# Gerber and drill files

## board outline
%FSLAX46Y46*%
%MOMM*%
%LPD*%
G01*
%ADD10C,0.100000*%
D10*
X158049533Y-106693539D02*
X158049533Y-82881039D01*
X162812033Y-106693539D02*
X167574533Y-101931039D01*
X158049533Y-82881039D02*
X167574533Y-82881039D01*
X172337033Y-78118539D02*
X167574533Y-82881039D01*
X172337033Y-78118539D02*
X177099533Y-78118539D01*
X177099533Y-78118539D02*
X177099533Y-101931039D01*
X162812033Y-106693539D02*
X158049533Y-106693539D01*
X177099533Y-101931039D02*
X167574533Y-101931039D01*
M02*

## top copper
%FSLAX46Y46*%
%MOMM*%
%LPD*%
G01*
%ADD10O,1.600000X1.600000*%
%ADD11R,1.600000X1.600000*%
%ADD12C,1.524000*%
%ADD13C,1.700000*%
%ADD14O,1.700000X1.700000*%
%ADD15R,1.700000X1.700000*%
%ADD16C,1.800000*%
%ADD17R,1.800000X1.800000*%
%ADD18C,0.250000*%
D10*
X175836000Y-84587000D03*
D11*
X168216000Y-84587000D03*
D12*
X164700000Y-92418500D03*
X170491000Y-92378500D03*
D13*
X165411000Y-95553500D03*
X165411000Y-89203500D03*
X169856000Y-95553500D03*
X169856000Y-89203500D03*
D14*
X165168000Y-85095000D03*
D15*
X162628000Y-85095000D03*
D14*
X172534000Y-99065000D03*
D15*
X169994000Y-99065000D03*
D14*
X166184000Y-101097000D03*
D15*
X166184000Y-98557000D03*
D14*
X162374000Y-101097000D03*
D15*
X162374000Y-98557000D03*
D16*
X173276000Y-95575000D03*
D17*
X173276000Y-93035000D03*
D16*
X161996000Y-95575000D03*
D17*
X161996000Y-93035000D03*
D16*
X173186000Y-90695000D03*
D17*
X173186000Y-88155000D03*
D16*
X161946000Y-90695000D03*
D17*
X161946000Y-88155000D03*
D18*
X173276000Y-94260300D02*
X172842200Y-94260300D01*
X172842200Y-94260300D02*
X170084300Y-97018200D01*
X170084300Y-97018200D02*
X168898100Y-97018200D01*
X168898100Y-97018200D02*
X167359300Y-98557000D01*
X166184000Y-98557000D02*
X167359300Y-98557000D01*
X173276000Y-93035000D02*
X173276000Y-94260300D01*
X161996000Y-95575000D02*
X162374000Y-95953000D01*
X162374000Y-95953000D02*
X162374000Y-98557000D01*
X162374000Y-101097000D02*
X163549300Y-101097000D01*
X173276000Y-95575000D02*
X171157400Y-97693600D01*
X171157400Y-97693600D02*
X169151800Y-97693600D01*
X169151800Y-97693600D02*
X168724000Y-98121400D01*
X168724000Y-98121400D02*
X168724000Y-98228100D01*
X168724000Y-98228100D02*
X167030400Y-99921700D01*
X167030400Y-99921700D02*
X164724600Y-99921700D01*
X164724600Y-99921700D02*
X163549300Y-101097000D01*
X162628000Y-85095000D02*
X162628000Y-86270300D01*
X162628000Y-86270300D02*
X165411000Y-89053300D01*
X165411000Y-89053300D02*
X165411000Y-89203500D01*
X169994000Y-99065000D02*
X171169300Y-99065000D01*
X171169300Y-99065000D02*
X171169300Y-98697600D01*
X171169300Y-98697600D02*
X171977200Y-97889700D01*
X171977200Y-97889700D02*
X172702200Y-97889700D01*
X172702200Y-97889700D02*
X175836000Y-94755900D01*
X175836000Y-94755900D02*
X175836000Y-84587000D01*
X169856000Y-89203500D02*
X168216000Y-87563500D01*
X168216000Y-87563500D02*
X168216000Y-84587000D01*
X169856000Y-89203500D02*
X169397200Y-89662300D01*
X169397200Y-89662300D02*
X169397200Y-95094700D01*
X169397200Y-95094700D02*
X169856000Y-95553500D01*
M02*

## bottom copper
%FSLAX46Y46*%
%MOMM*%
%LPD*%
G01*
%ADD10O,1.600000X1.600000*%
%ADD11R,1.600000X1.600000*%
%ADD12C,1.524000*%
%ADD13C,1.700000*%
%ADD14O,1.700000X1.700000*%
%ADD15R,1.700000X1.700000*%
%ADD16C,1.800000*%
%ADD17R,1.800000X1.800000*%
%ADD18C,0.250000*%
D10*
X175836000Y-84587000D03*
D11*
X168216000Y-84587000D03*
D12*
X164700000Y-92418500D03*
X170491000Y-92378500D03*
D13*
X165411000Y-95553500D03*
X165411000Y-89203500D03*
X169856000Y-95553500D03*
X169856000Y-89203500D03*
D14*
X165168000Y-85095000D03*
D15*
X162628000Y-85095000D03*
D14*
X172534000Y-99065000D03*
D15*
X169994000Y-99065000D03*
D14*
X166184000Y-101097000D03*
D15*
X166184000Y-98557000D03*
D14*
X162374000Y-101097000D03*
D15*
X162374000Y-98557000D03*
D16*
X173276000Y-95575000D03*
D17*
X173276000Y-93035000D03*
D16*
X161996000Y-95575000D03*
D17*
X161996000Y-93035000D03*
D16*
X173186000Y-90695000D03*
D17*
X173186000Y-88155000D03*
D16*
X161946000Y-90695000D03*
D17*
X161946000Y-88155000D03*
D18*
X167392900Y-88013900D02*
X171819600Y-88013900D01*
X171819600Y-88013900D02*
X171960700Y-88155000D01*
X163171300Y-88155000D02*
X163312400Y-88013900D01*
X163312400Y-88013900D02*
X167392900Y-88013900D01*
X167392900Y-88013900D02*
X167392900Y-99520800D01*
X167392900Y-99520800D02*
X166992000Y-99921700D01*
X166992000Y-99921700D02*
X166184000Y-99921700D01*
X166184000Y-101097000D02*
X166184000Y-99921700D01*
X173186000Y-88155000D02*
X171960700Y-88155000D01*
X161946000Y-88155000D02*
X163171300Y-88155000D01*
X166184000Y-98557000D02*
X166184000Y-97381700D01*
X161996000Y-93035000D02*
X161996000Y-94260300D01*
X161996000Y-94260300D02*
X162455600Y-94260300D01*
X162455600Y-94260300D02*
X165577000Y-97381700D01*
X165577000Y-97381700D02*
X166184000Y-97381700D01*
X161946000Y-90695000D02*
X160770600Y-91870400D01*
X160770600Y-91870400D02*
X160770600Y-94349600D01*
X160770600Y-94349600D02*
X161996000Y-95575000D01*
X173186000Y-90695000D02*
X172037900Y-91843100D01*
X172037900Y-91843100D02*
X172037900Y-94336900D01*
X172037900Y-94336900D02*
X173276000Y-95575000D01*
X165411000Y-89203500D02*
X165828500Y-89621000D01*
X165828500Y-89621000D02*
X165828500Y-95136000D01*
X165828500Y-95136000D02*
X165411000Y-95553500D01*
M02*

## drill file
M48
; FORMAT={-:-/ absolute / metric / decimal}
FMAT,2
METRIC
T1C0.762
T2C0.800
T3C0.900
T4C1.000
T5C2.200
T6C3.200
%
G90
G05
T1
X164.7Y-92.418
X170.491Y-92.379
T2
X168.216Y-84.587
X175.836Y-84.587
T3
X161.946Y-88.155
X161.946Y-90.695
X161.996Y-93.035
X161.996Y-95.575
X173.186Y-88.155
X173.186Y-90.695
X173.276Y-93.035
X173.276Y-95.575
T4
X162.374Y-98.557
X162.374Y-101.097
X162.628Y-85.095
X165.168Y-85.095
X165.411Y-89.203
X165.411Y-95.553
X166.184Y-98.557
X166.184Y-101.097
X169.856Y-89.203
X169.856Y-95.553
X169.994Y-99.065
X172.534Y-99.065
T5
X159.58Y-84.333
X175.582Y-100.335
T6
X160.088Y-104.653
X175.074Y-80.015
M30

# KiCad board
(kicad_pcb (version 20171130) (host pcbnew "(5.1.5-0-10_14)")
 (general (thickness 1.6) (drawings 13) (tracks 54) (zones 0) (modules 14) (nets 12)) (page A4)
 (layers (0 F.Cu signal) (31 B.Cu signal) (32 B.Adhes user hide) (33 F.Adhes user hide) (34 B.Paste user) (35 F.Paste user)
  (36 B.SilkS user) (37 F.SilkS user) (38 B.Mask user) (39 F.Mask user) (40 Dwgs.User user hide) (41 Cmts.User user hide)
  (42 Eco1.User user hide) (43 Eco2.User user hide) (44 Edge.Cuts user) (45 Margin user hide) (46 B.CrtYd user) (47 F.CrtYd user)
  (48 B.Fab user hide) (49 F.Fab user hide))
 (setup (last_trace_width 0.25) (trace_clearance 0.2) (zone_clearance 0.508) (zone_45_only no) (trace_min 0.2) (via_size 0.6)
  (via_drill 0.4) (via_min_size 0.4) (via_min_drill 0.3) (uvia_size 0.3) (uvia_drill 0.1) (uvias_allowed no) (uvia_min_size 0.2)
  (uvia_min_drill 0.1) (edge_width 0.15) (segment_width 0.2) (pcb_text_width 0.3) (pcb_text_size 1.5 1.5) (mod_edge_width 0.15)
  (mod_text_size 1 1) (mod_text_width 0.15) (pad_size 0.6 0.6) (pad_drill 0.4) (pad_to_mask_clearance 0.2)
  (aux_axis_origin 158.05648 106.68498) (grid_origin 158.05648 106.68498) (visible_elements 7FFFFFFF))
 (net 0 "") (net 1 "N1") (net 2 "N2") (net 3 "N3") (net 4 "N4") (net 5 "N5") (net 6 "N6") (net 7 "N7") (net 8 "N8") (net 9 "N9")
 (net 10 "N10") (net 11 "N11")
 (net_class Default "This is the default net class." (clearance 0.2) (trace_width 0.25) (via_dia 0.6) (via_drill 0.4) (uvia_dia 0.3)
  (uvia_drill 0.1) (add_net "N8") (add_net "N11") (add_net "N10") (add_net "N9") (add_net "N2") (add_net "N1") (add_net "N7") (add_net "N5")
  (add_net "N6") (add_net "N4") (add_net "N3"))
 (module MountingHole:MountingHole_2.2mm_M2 (layer F.Cu) (at 159.58048 84.33298)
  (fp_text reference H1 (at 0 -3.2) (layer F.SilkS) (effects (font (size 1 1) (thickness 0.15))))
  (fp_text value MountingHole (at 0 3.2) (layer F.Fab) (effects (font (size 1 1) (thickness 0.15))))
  (pad 1 np_thru_hole circle (at 0 0) (size 2.2 2.2) (drill 2.2) (layers *.Cu *.Mask)))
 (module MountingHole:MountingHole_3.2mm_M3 (layer F.Cu) (at 160.08848 104.65298)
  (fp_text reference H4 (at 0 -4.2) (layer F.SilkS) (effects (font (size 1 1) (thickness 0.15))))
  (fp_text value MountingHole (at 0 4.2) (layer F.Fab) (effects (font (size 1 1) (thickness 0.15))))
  (pad 1 np_thru_hole circle (at 0 0) (size 3.2 3.2) (drill 3.2) (layers *.Cu *.Mask)))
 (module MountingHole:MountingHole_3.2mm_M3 (layer F.Cu) (at 175.07448 80.01498)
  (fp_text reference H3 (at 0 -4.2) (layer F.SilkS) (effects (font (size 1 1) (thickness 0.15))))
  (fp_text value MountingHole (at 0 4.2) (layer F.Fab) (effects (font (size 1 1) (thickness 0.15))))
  (pad 1 np_thru_hole circle (at 0 0) (size 3.2 3.2) (drill 3.2) (layers *.Cu *.Mask)))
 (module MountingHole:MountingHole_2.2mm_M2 (layer F.Cu) (at 175.58248 100.33498)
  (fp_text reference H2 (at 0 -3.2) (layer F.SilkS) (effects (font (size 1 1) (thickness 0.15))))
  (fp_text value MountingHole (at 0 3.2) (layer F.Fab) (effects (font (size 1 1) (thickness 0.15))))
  (pad 1 np_thru_hole circle (at 0 0) (size 2.2 2.2) (drill 2.2) (layers *.Cu *.Mask)))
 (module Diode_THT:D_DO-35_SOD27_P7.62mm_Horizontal (layer F.Cu) (at 168.216 84.587)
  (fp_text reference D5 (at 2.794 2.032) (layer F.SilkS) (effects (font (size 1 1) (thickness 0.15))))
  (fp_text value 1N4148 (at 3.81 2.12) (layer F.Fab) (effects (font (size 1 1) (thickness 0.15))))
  (pad 2 thru_hole oval (at 7.62 0) (size 1.6 1.6) (drill 0.8) (layers *.Cu *.Mask) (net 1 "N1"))
  (pad 1 thru_hole rect (at 0 0) (size 1.6 1.6) (drill 0.8) (layers *.Cu *.Mask) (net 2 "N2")))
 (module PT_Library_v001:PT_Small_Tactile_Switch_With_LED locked (layer F.Cu) (at 167.57 92.3785 270)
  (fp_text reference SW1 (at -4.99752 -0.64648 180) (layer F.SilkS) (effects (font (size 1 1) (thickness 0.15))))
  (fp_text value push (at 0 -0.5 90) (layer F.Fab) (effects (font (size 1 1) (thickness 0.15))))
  (pad 6 thru_hole circle (at 0.04 2.87 270) (size 1.524 1.524) (drill 0.762) (layers *.Cu *.Mask) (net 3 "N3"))
  (pad 5 thru_hole circle (at 0 -2.921 270) (size 1.524 1.524) (drill 0.762) (layers *.Cu *.Mask) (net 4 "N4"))
  (pad 4 thru_hole circle (at 3.175 2.159 270) (size 1.7 1.7) (drill 1) (layers *.Cu *.Mask) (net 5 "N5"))
  (pad 3 thru_hole circle (at -3.175 2.159 270) (size 1.7 1.7) (drill 1) (layers *.Cu *.Mask) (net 5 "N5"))
  (pad 2 thru_hole circle (at 3.175 -2.286 270) (size 1.7 1.7) (drill 1) (layers *.Cu *.Mask) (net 2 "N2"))
  (pad 1 thru_hole circle (at -3.175 -2.286 270) (size 1.7 1.7) (drill 1) (layers *.Cu *.Mask) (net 2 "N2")))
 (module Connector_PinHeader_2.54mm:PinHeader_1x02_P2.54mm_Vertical (layer B.Cu) (at 162.628 85.095 270)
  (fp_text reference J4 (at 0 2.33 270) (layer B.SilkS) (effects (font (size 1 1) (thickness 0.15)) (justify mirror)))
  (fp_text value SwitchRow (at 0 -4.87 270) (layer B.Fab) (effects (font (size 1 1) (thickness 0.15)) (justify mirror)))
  (pad 2 thru_hole oval (at 0 -2.54 270) (size 1.7 1.7) (drill 1) (layers *.Cu *.Mask) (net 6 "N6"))
  (pad 1 thru_hole rect (at 0 0 270) (size 1.7 1.7) (drill 1) (layers *.Cu *.Mask) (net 5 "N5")))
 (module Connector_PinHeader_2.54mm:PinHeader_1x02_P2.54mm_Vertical (layer B.Cu) (at 169.994 99.065 270)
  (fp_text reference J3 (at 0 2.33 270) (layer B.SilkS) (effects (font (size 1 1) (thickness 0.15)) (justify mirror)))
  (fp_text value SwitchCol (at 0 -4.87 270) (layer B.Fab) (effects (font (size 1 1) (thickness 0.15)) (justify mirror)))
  (pad 2 thru_hole oval (at 0 -2.54 270) (size 1.7 1.7) (drill 1) (layers *.Cu *.Mask) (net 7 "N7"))
  (pad 1 thru_hole rect (at 0 0 270) (size 1.7 1.7) (drill 1) (layers *.Cu *.Mask) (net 1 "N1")))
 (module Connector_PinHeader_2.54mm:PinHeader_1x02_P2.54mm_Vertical (layer B.Cu) (at 166.184 98.557 180)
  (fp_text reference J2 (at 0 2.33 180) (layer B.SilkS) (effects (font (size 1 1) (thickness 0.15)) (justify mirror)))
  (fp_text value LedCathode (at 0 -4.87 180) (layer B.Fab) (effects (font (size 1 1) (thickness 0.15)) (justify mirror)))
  (pad 2 thru_hole oval (at 0 -2.54 180) (size 1.7 1.7) (drill 1) (layers *.Cu *.Mask) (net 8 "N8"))
  (pad 1 thru_hole rect (at 0 0 180) (size 1.7 1.7) (drill 1) (layers *.Cu *.Mask) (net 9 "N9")))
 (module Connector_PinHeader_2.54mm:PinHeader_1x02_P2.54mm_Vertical (layer B.Cu) (at 162.374 98.557 180)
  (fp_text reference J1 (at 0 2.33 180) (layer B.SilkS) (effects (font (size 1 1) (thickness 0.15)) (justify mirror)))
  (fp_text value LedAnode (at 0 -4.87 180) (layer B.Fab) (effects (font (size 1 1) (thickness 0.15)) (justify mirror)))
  (pad 2 thru_hole oval (at 0 -2.54 180) (size 1.7 1.7) (drill 1) (layers *.Cu *.Mask) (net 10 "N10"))
  (pad 1 thru_hole rect (at 0 0 180) (size 1.7 1.7) (drill 1) (layers *.Cu *.Mask) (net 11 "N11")))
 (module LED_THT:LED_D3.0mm (layer F.Cu) (at 173.276 93.035 270)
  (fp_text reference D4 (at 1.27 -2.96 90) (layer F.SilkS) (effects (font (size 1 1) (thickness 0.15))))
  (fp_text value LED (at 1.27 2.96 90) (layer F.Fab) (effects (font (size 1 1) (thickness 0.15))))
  (pad 2 thru_hole circle (at 2.54 0 270) (size 1.8 1.8) (drill 0.9) (layers *.Cu *.Mask) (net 10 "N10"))
  (pad 1 thru_hole rect (at 0 0 270) (size 1.8 1.8) (drill 0.9) (layers *.Cu *.Mask) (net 9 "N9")))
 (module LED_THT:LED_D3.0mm (layer F.Cu) (at 161.996 93.035 270)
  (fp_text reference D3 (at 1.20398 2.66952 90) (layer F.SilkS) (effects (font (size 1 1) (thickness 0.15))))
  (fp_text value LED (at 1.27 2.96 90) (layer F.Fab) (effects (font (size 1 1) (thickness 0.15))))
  (pad 2 thru_hole circle (at 2.54 0 270) (size 1.8 1.8) (drill 0.9) (layers *.Cu *.Mask) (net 11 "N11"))
  (pad 1 thru_hole rect (at 0 0 270) (size 1.8 1.8) (drill 0.9) (layers *.Cu *.Mask) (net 9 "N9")))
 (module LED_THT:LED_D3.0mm (layer F.Cu) (at 173.186 88.155 270)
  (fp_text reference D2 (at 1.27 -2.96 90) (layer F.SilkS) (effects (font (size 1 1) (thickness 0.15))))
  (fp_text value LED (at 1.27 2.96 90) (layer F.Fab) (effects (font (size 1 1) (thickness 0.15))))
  (pad 2 thru_hole circle (at 2.54 0 270) (size 1.8 1.8) (drill 0.9) (layers *.Cu *.Mask) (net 10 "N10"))
  (pad 1 thru_hole rect (at 0 0 270) (size 1.8 1.8) (drill 0.9) (layers *.Cu *.Mask) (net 8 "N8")))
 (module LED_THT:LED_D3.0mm (layer F.Cu) (at 161.946 88.155 270)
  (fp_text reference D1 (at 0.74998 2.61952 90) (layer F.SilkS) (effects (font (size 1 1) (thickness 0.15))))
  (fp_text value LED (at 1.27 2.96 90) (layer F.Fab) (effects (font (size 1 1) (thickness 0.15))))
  (pad 2 thru_hole circle (at 2.54 0 270) (size 1.8 1.8) (drill 0.9) (layers *.Cu *.Mask) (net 11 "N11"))
  (pad 1 thru_hole rect (at 0 0 270) (size 1.8 1.8) (drill 0.9) (layers *.Cu *.Mask) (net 8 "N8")))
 (gr_line (start 158.049533 106.693539) (end 158.049533 82.881039) (layer Edge.Cuts) (width 0.1))
 (gr_line (start 162.812033 106.693539) (end 167.574533 101.931039) (layer Edge.Cuts) (width 0.1))
 (gr_line (start 158.049533 82.881039) (end 167.574533 82.881039) (layer Edge.Cuts) (width 0.1))
 (gr_line (start 172.337033 78.118539) (end 167.574533 82.881039) (layer Edge.Cuts) (width 0.1))
 (gr_line (start 172.337033 78.118539) (end 177.099533 78.118539) (layer Edge.Cuts) (width 0.1))
 (gr_line (start 177.099533 78.118539) (end 177.099533 101.931039) (layer Edge.Cuts) (width 0.1))
 (gr_line (start 162.812033 106.693539) (end 158.049533 106.693539) (layer Edge.Cuts) (width 0.1))
 (gr_line (start 177.099533 101.931039) (end 167.574533 101.931039) (layer Edge.Cuts) (width 0.1))
 (segment (start 167.3929 88.0139) (end 171.8196 88.0139) (width 0.25) (layer B.Cu) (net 8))
 (segment (start 171.8196 88.0139) (end 171.9607 88.155) (width 0.25) (layer B.Cu) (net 8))
 (segment (start 163.1713 88.155) (end 163.3124 88.0139) (width 0.25) (layer B.Cu) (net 8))
 (segment (start 163.3124 88.0139) (end 167.3929 88.0139) (width 0.25) (layer B.Cu) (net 8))
 (segment (start 167.3929 88.0139) (end 167.3929 99.5208) (width 0.25) (layer B.Cu) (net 8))
 (segment (start 167.3929 99.5208) (end 166.992 99.9217) (width 0.25) (layer B.Cu) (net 8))
 (segment (start 166.992 99.9217) (end 166.184 99.9217) (width 0.25) (layer B.Cu) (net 8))
 (segment (start 166.184 101.097) (end 166.184 99.9217) (width 0.25) (layer B.Cu) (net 8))
 (segment (start 173.186 88.155) (end 171.9607 88.155) (width 0.25) (layer B.Cu) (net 8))
 (segment (start 161.946 88.155) (end 163.1713 88.155) (width 0.25) (layer B.Cu) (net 8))
 (segment (start 173.276 94.2603) (end 172.8422 94.2603) (width 0.25) (layer F.Cu) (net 9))
 (segment (start 172.8422 94.2603) (end 170.0843 97.0182) (width 0.25) (layer F.Cu) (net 9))
 (segment (start 170.0843 97.0182) (end 168.8981 97.0182) (width 0.25) (layer F.Cu) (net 9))
 (segment (start 168.8981 97.0182) (end 167.3593 98.557) (width 0.25) (layer F.Cu) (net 9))
 (segment (start 166.184 98.557) (end 167.3593 98.557) (width 0.25) (layer F.Cu) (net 9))
 (segment (start 173.276 93.035) (end 173.276 94.2603) (width 0.25) (layer F.Cu) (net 9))
 (segment (start 166.184 98.557) (end 166.184 97.3817) (width 0.25) (layer B.Cu) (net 9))
 (segment (start 161.996 93.035) (end 161.996 94.2603) (width 0.25) (layer B.Cu) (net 9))
 (segment (start 161.996 94.2603) (end 162.4556 94.2603) (width 0.25) (layer B.Cu) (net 9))
 (segment (start 162.4556 94.2603) (end 165.577 97.3817) (width 0.25) (layer B.Cu) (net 9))
 (segment (start 165.577 97.3817) (end 166.184 97.3817) (width 0.25) (layer B.Cu) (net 9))
 (segment (start 161.996 95.575) (end 162.374 95.953) (width 0.25) (layer F.Cu) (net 11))
 (segment (start 162.374 95.953) (end 162.374 98.557) (width 0.25) (layer F.Cu) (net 11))
 (segment (start 161.946 90.695) (end 160.7706 91.8704) (width 0.25) (layer B.Cu) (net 11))
 (segment (start 160.7706 91.8704) (end 160.7706 94.3496) (width 0.25) (layer B.Cu) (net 11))
 (segment (start 160.7706 94.3496) (end 161.996 95.575) (width 0.25) (layer B.Cu) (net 11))
 (segment (start 162.374 101.097) (end 163.5493 101.097) (width 0.25) (layer F.Cu) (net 10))
 (segment (start 173.276 95.575) (end 171.1574 97.6936) (width 0.25) (layer F.Cu) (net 10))
 (segment (start 171.1574 97.6936) (end 169.1518 97.6936) (width 0.25) (layer F.Cu) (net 10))
 (segment (start 169.1518 97.6936) (end 168.724 98.1214) (width 0.25) (layer F.Cu) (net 10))
 (segment (start 168.724 98.1214) (end 168.724 98.2281) (width 0.25) (layer F.Cu) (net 10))
 (segment (start 168.724 98.2281) (end 167.0304 99.9217) (width 0.25) (layer F.Cu) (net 10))
 (segment (start 167.0304 99.9217) (end 164.7246 99.9217) (width 0.25) (layer F.Cu) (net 10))
 (segment (start 164.7246 99.9217) (end 163.5493 101.097) (width 0.25) (layer F.Cu) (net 10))
 (segment (start 173.186 90.695) (end 172.0379 91.8431) (width 0.25) (layer B.Cu) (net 10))
 (segment (start 172.0379 91.8431) (end 172.0379 94.3369) (width 0.25) (layer B.Cu) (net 10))
 (segment (start 172.0379 94.3369) (end 173.276 95.575) (width 0.25) (layer B.Cu) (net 10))
 (segment (start 162.628 85.095) (end 162.628 86.2703) (width 0.25) (layer F.Cu) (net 5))
 (segment (start 162.628 86.2703) (end 165.411 89.0533) (width 0.25) (layer F.Cu) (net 5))
 (segment (start 165.411 89.0533) (end 165.411 89.2035) (width 0.25) (layer F.Cu) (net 5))
 (segment (start 165.411 89.2035) (end 165.8285 89.621) (width 0.25) (layer B.Cu) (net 5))
 (segment (start 165.8285 89.621) (end 165.8285 95.136) (width 0.25) (layer B.Cu) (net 5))
 (segment (start 165.8285 95.136) (end 165.411 95.5535) (width 0.25) (layer B.Cu) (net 5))
 (segment (start 169.994 99.065) (end 171.1693 99.065) (width 0.25) (layer F.Cu) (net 1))
 (segment (start 171.1693 99.065) (end 171.1693 98.6976) (width 0.25) (layer F.Cu) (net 1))
 (segment (start 171.1693 98.6976) (end 171.9772 97.8897) (width 0.25) (layer F.Cu) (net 1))
 (segment (start 171.9772 97.8897) (end 172.7022 97.8897) (width 0.25) (layer F.Cu) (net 1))
 (segment (start 172.7022 97.8897) (end 175.836 94.7559) (width 0.25) (layer F.Cu) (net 1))
 (segment (start 175.836 94.7559) (end 175.836 84.587) (width 0.25) (layer F.Cu) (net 1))
 (segment (start 169.856 89.2035) (end 168.216 87.5635) (width 0.25) (layer F.Cu) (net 2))
 (segment (start 168.216 87.5635) (end 168.216 84.587) (width 0.25) (layer F.Cu) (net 2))
 (segment (start 169.856 89.2035) (end 169.3972 89.6623) (width 0.25) (layer F.Cu) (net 2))
 (segment (start 169.3972 89.6623) (end 169.3972 95.0947) (width 0.25) (layer F.Cu) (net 2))
 (segment (start 169.3972 95.0947) (end 169.856 95.5535) (width 0.25) (layer F.Cu) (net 2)))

